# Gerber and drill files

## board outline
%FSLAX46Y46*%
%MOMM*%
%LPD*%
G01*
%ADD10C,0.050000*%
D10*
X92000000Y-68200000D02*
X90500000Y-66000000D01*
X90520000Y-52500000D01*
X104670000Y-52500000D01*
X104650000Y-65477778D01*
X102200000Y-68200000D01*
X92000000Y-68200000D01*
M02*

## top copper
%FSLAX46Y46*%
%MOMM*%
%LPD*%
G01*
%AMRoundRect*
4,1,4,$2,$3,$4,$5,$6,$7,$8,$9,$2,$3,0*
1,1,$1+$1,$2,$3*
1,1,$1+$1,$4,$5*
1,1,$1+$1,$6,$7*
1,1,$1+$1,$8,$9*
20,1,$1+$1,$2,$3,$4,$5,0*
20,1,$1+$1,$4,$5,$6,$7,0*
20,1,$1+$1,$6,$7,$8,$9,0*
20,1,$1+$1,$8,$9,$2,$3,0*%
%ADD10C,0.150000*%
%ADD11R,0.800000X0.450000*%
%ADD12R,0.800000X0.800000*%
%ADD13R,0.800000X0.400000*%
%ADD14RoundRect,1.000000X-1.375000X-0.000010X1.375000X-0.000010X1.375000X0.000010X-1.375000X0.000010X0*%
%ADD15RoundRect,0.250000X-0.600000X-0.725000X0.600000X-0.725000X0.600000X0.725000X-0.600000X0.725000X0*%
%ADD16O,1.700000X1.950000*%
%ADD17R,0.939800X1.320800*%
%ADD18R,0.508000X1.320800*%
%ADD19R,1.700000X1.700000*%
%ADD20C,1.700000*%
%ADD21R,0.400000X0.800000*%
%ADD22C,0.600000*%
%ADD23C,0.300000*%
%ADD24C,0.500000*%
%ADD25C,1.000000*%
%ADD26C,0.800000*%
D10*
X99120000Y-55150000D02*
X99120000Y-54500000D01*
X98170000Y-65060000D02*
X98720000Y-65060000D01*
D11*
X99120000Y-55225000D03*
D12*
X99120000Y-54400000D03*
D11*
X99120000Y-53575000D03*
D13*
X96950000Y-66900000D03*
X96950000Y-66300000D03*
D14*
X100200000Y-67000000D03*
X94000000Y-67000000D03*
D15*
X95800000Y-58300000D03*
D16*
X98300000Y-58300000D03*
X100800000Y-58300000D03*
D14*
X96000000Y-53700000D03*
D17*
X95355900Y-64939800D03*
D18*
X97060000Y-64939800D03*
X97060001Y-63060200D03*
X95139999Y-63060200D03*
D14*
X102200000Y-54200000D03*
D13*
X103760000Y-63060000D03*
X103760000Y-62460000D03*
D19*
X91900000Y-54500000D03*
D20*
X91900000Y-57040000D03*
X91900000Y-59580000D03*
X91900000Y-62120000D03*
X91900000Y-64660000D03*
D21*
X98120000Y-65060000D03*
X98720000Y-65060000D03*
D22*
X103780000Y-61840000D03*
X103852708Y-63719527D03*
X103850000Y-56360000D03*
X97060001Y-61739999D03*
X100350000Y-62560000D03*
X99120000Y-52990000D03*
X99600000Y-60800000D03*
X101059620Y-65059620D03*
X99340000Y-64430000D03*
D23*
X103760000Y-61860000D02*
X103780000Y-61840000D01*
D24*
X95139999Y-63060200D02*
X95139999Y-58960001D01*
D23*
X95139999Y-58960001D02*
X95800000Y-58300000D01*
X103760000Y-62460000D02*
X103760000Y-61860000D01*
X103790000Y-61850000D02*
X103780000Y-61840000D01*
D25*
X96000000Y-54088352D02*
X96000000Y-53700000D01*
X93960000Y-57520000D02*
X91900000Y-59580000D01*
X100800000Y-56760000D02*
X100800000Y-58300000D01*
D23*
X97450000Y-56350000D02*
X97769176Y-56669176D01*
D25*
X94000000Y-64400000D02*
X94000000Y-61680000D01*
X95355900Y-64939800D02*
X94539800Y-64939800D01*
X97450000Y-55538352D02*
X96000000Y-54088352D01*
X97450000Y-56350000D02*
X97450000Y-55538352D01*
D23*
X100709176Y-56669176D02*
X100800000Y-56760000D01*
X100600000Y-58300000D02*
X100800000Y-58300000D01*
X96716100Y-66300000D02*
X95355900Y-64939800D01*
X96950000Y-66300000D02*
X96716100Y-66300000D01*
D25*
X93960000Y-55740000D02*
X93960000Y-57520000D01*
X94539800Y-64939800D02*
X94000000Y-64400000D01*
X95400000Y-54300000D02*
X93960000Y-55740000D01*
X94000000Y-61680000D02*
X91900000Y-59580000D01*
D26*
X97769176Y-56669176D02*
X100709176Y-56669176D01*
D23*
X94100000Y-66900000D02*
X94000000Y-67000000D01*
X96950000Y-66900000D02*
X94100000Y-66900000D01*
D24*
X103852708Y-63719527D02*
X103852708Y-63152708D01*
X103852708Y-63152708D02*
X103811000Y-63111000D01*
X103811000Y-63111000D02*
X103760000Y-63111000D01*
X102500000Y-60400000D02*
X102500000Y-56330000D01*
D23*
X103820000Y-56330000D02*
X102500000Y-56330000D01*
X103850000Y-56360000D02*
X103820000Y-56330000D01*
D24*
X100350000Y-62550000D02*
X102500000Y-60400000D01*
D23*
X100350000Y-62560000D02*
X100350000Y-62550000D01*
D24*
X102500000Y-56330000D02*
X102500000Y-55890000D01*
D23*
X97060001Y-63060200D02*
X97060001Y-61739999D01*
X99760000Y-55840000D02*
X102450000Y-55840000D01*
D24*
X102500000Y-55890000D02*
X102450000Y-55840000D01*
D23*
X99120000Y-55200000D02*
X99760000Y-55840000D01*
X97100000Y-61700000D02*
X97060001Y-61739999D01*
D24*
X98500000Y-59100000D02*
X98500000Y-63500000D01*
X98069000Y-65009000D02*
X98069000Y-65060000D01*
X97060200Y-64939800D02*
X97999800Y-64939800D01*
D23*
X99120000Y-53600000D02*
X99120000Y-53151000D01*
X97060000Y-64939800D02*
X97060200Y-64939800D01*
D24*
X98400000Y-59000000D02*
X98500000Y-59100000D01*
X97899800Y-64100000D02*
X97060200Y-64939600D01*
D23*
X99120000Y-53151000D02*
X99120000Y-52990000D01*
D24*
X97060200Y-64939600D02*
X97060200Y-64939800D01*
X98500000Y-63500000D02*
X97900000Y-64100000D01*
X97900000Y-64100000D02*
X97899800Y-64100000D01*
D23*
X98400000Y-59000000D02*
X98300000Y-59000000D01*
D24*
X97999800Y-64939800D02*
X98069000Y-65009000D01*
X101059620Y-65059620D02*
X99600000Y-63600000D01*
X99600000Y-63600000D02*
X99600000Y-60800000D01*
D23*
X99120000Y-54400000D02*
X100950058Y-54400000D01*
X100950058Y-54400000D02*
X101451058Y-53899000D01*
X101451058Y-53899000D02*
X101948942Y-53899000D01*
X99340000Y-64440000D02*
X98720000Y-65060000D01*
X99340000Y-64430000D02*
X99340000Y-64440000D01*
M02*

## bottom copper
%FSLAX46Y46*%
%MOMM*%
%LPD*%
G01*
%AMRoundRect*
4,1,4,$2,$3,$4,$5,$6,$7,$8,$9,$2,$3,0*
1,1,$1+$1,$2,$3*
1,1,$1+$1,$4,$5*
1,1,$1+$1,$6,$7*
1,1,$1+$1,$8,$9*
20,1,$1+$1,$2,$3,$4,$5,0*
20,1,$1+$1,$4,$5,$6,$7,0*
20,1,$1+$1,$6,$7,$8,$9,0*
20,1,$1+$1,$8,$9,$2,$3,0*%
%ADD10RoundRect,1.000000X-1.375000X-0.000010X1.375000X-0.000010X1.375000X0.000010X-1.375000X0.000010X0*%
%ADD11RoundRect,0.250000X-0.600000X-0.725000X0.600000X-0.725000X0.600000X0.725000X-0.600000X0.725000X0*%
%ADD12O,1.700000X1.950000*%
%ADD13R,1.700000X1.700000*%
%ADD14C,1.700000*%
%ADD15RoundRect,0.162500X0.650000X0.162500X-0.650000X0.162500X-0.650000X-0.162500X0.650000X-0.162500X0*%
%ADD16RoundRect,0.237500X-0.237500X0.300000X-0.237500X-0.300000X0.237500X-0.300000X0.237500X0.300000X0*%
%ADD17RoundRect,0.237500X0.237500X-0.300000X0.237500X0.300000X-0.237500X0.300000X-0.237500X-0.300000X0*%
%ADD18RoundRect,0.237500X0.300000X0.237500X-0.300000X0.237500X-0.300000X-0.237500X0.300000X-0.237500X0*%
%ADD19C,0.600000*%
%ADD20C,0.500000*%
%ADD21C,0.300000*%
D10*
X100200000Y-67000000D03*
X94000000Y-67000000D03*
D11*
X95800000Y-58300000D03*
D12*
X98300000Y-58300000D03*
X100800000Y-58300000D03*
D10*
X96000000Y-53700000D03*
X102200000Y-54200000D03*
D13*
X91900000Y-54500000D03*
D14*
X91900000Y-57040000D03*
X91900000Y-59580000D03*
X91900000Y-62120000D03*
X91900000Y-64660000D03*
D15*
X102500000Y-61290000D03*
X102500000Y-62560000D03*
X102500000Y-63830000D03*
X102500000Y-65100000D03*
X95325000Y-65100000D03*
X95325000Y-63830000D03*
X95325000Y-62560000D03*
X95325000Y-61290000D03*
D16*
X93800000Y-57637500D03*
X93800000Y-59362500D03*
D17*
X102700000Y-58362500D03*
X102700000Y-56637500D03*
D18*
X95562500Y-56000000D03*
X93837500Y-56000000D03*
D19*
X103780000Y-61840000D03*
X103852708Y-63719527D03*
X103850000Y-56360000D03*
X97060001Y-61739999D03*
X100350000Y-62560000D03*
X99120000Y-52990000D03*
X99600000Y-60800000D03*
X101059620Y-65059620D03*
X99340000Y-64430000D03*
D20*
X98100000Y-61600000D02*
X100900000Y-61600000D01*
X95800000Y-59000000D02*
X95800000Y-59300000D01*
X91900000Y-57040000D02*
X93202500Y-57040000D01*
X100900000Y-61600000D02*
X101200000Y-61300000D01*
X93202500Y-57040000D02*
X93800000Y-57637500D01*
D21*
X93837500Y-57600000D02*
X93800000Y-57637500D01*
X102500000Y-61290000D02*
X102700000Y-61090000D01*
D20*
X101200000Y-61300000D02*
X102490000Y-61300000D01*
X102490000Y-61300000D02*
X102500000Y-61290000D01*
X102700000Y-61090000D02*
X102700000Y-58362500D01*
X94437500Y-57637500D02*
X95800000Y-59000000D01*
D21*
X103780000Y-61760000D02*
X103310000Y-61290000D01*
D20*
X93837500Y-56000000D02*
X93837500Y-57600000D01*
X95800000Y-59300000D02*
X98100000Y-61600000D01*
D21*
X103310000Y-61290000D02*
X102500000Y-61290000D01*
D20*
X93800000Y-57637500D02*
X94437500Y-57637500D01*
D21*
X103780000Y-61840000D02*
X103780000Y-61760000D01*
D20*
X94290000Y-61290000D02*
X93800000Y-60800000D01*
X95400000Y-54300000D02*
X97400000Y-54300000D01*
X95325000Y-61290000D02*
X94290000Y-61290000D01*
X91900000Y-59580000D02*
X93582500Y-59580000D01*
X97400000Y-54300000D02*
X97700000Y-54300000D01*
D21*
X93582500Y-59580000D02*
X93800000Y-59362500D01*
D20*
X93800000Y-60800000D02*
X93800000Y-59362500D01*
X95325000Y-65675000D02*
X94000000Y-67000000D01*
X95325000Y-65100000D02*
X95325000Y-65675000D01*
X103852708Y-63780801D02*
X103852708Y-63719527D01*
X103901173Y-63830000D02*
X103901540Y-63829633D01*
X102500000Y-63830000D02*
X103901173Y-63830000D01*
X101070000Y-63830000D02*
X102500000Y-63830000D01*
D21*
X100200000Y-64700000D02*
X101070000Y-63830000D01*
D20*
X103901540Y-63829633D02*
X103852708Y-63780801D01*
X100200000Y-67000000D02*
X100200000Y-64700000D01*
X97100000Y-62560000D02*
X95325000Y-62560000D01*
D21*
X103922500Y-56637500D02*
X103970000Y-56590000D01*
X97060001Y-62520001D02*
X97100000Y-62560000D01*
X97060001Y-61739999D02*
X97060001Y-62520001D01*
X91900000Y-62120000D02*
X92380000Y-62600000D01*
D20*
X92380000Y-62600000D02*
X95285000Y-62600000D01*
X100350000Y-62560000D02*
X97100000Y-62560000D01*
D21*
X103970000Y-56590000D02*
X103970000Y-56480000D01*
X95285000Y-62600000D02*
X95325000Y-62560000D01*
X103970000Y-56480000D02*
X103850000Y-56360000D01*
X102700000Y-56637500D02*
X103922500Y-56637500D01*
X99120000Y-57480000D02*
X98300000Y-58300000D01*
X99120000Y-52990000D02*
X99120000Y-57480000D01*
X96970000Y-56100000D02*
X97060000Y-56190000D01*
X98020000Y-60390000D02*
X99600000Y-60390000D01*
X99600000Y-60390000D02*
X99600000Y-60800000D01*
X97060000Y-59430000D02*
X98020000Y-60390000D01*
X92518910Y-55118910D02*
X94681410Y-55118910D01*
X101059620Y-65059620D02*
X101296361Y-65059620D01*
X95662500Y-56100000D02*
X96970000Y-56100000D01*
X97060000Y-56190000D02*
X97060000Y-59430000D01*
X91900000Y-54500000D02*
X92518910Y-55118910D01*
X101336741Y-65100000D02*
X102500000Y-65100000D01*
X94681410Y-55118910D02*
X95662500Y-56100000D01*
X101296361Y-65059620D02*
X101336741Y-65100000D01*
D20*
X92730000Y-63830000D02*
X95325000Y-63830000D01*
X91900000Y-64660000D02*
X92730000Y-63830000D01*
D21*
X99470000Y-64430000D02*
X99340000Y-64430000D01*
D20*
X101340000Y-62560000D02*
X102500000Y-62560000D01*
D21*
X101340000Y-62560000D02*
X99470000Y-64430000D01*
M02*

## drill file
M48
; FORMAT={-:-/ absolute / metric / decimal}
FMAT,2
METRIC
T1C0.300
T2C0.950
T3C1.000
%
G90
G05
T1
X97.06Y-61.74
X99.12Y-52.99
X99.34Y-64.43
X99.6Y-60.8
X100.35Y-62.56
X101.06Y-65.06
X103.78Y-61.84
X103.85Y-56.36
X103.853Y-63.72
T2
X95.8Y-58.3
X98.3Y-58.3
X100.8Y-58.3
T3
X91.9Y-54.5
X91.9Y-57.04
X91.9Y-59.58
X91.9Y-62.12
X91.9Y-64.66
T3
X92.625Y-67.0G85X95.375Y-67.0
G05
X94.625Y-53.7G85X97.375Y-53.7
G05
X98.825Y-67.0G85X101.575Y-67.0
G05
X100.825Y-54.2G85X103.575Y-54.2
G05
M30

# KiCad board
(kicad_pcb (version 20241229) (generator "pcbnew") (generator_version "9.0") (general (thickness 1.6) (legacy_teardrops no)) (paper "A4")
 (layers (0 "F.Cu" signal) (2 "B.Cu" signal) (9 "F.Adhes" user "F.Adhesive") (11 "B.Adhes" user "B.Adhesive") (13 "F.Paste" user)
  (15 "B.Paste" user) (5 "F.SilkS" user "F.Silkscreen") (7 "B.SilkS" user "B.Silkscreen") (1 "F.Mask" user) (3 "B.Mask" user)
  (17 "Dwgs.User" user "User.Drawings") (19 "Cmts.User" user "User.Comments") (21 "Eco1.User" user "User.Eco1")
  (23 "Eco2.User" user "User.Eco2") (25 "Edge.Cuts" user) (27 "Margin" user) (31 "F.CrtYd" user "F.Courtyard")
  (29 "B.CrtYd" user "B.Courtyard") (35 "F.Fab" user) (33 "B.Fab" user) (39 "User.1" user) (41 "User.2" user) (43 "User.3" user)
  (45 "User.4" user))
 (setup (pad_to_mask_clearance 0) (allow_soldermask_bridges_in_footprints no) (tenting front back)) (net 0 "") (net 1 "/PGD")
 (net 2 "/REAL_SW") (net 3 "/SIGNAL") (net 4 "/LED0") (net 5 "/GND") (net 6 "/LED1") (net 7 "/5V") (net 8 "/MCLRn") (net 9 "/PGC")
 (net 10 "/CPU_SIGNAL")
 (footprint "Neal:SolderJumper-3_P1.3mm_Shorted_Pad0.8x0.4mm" (layer "F.Cu") (at 99.12 54.4 90)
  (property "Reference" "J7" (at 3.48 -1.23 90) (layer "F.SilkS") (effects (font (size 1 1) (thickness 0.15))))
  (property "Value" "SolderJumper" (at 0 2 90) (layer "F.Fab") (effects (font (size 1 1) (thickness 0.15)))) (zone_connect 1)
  (fp_line (start -0.75 0) (end -0.1 0) (stroke (width 0.15) (type solid)) (layer "F.Cu"))
  (pad "1" smd rect (at -0.825 0 90) (size 0.45 0.8) (layers "F.Cu" "F.Mask") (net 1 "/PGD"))
  (pad "2" smd rect (at 0 0 90) (size 0.8 0.8) (layers "F.Cu" "F.Mask") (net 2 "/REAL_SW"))
  (pad "3" smd rect (at 0.825 0 90) (size 0.45 0.8) (layers "F.Cu" "F.Mask") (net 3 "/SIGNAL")))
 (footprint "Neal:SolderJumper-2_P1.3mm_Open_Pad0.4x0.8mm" (layer "F.Cu") (at 96.95 66.6 90)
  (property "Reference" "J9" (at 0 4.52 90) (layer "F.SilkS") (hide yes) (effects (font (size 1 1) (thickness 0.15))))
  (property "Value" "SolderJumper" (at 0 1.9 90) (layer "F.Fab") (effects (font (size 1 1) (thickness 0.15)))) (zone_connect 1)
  (pad "1" smd rect (at -0.3 0 90) (size 0.4 0.8) (layers "F.Cu" "F.Mask") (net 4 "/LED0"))
  (pad "2" smd rect (at 0.3 0 90) (size 0.4 0.8) (layers "F.Cu" "F.Mask") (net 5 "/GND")))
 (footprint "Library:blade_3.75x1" (layer "F.Cu") (at 100.2 67)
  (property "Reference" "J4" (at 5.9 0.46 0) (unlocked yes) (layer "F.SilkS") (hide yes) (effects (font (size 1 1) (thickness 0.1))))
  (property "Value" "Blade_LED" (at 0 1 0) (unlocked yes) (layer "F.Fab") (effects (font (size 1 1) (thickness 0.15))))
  (pad "1" thru_hole roundrect (at 0 0) (size 4.75 2) (drill oval 3.75 1) (layers "*.Cu" "*.Mask") (remove_unused_layers no)
   (roundrect_rratio 0.5) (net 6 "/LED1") (thermal_bridge_angle 45)))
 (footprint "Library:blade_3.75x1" (layer "F.Cu") (at 94 67)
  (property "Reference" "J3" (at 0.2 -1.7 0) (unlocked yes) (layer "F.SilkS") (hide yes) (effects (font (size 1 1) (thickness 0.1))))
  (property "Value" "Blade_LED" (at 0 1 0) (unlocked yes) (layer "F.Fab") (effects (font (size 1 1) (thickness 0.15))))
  (pad "1" thru_hole roundrect (at 0 0) (size 4.75 2) (drill oval 3.75 1) (layers "*.Cu" "*.Mask") (remove_unused_layers no)
   (roundrect_rratio 0.5) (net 4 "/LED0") (thermal_bridge_angle 45)))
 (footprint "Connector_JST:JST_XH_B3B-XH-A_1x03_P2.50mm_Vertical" (layer "F.Cu") (at 95.8 58.3)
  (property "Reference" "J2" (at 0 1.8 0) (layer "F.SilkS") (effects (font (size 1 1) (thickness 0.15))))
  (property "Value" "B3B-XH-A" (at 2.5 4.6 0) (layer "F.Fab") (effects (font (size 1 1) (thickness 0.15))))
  (pad "1" thru_hole roundrect (at 0 0) (size 1.7 1.95) (drill 0.95) (layers "*.Cu" "*.Mask") (remove_unused_layers no)
   (roundrect_rratio 0.147059) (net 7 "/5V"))
  (pad "2" thru_hole oval (at 2.5 0) (size 1.7 1.95) (drill 0.95) (layers "*.Cu" "*.Mask") (remove_unused_layers no) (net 3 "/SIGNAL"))
  (pad "3" thru_hole oval (at 5 0) (size 1.7 1.95) (drill 0.95) (layers "*.Cu" "*.Mask") (remove_unused_layers no) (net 5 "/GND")))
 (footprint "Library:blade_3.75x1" (layer "F.Cu") (at 95.4 54.3)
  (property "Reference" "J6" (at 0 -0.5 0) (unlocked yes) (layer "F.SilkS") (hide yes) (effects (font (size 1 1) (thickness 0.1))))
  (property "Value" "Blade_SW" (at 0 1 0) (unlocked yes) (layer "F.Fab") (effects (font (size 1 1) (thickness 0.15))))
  (pad "1" thru_hole roundrect (at 0.6 -0.6) (size 4.75 2) (drill oval 3.75 1) (layers "*.Cu" "*.Mask") (remove_unused_layers no)
   (roundrect_rratio 0.5) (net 5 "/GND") (thermal_bridge_angle 45)))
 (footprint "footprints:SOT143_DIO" (layer "F.Cu") (at 96.1 64)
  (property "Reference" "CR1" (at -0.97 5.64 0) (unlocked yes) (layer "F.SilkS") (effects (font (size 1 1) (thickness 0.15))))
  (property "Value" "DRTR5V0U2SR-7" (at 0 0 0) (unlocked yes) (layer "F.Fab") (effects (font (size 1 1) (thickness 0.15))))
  (pad "1" smd rect (at -0.7441 0.9398) (size 0.9398 1.3208) (layers "F.Cu" "F.Mask" "F.Paste") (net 5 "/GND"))
  (pad "2" smd rect (at 0.96 0.9398) (size 0.508 1.3208) (layers "F.Cu" "F.Mask" "F.Paste") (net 3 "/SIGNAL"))
  (pad "3" smd rect (at 0.960001 -0.9398) (size 0.508 1.3208) (layers "F.Cu" "F.Mask" "F.Paste") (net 1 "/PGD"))
  (pad "4" smd rect (at -0.960001 -0.9398) (size 0.508 1.3208) (layers "F.Cu" "F.Mask" "F.Paste") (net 7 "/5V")))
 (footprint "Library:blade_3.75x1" (layer "F.Cu") (at 101.7 55.5)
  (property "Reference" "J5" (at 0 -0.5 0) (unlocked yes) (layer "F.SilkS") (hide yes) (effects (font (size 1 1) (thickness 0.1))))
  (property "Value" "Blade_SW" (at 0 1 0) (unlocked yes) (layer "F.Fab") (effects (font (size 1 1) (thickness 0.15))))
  (pad "1" thru_hole roundrect (at 0.5 -1.3) (size 4.75 2) (drill oval 3.75 1) (layers "*.Cu" "*.Mask") (remove_unused_layers no)
   (roundrect_rratio 0.5) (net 2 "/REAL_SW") (thermal_bridge_angle 45)))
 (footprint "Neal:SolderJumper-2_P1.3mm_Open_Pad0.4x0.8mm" (layer "F.Cu") (at 103.76 62.76 90)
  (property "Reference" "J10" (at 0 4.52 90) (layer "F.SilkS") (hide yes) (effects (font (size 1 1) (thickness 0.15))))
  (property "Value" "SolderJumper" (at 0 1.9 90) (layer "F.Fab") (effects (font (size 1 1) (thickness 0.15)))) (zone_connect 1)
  (pad "1" smd rect (at -0.3 0 90) (size 0.4 0.8) (layers "F.Cu" "F.Mask") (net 6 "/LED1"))
  (pad "2" smd rect (at 0.3 0 90) (size 0.4 0.8) (layers "F.Cu" "F.Mask") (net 7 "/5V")))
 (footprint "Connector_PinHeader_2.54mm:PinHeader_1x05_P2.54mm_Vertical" (layer "F.Cu") (at 91.9 54.5)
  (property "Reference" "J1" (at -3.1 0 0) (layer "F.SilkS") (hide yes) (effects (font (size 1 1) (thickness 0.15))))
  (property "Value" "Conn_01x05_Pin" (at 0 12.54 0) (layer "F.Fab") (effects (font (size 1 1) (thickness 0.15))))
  (pad "1" thru_hole rect (at 0 0) (size 1.7 1.7) (drill 1) (layers "*.Cu" "*.Mask") (remove_unused_layers no) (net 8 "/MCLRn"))
  (pad "2" thru_hole circle (at 0 2.54) (size 1.7 1.7) (drill 1) (layers "*.Cu" "*.Mask") (remove_unused_layers no) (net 7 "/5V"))
  (pad "3" thru_hole circle (at 0 5.08) (size 1.7 1.7) (drill 1) (layers "*.Cu" "*.Mask") (remove_unused_layers no) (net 5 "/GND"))
  (pad "4" thru_hole circle (at 0 7.62) (size 1.7 1.7) (drill 1) (layers "*.Cu" "*.Mask") (remove_unused_layers no) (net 1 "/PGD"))
  (pad "5" thru_hole circle (at 0 10.16) (size 1.7 1.7) (drill 1) (layers "*.Cu" "*.Mask") (remove_unused_layers no) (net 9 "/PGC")))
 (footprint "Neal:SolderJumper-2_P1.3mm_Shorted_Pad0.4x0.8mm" (layer "F.Cu") (at 98.42 65.06)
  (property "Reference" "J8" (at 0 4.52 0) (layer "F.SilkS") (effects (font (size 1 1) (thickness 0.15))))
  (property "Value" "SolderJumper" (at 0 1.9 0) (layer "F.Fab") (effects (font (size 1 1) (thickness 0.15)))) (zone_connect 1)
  (fp_line (start -0.25 0) (end 0.3 0) (stroke (width 0.15) (type solid)) (layer "F.Cu"))
  (pad "1" smd rect (at -0.3 0) (size 0.4 0.8) (layers "F.Cu" "F.Mask") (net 3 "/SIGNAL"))
  (pad "2" smd rect (at 0.3 0) (size 0.4 0.8) (layers "F.Cu" "F.Mask") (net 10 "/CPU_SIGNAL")))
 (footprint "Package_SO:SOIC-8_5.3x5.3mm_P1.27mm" (layer "B.Cu") (at 98.9125 63.195 180)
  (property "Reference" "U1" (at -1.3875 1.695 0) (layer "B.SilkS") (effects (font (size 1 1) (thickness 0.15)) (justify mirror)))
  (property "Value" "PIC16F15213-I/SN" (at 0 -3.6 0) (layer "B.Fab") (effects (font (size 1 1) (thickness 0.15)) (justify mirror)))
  (pad "1" smd roundrect (at -3.5875 1.905 180) (size 1.625 0.65) (layers "B.Cu" "B.Mask" "B.Paste") (roundrect_rratio 0.25) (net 7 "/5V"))
  (pad "2" smd roundrect (at -3.5875 0.635 180) (size 1.625 0.65) (layers "B.Cu" "B.Mask" "B.Paste") (roundrect_rratio 0.25)
   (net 10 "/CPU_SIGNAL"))
  (pad "3" smd roundrect (at -3.5875 -0.635 180) (size 1.625 0.65) (layers "B.Cu" "B.Mask" "B.Paste") (roundrect_rratio 0.25)
   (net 6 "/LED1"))
  (pad "4" smd roundrect (at -3.5875 -1.905 180) (size 1.625 0.65) (layers "B.Cu" "B.Mask" "B.Paste") (roundrect_rratio 0.25)
   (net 8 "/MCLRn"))
  (pad "5" smd roundrect (at 3.5875 -1.905 180) (size 1.625 0.65) (layers "B.Cu" "B.Mask" "B.Paste") (roundrect_rratio 0.25) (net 4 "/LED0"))
  (pad "6" smd roundrect (at 3.5875 -0.635 180) (size 1.625 0.65) (layers "B.Cu" "B.Mask" "B.Paste") (roundrect_rratio 0.25) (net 9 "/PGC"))
  (pad "7" smd roundrect (at 3.5875 0.635 180) (size 1.625 0.65) (layers "B.Cu" "B.Mask" "B.Paste") (roundrect_rratio 0.25) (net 1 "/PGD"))
  (pad "8" smd roundrect (at 3.5875 1.905 180) (size 1.625 0.65) (layers "B.Cu" "B.Mask" "B.Paste") (roundrect_rratio 0.25) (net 5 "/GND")))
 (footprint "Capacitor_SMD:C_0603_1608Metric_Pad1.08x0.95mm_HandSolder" (layer "B.Cu") (at 93.8 58.5 -90)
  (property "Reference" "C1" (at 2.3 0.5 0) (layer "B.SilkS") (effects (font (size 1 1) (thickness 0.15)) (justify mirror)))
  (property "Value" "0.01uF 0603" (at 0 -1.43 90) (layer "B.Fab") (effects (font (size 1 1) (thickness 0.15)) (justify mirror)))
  (pad "1" smd roundrect (at -0.8625 0 270) (size 1.075 0.95) (layers "B.Cu" "B.Mask" "B.Paste") (roundrect_rratio 0.25) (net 7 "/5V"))
  (pad "2" smd roundrect (at 0.8625 0 270) (size 1.075 0.95) (layers "B.Cu" "B.Mask" "B.Paste") (roundrect_rratio 0.25) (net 5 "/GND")))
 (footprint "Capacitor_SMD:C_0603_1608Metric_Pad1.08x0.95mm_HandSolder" (layer "B.Cu") (at 102.7 57.5 90)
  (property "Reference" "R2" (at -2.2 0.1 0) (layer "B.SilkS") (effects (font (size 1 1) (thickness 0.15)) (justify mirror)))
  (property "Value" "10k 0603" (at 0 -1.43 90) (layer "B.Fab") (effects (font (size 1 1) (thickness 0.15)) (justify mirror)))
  (pad "1" smd roundrect (at -0.8625 0 90) (size 1.075 0.95) (layers "B.Cu" "B.Mask" "B.Paste") (roundrect_rratio 0.25) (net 7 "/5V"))
  (pad "2" smd roundrect (at 0.8625 0 90) (size 1.075 0.95) (layers "B.Cu" "B.Mask" "B.Paste") (roundrect_rratio 0.25) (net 1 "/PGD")))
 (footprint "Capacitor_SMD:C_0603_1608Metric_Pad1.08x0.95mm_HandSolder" (layer "B.Cu") (at 94.7 56 180)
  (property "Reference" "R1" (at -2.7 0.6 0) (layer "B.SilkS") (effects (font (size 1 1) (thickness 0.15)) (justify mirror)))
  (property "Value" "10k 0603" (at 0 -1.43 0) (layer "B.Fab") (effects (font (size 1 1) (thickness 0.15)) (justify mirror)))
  (pad "1" smd roundrect (at -0.8625 0 180) (size 1.075 0.95) (layers "B.Cu" "B.Mask" "B.Paste") (roundrect_rratio 0.25) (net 8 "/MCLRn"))
  (pad "2" smd roundrect (at 0.8625 0 180) (size 1.075 0.95) (layers "B.Cu" "B.Mask" "B.Paste") (roundrect_rratio 0.25) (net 7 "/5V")))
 (gr_poly
  (pts (xy 92 68.2) (xy 90.5 66) (xy 90.52 52.5) (xy 104.67 52.5) (xy 104.65 65.477778) (xy 102.2 68.2)) (stroke (width 0.05) (type solid))
  (fill no) (layer "Edge.Cuts"))
 (segment (start 103.76 61.86) (end 103.78 61.84) (width 0.3) (layer "F.Cu") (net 7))
 (segment (start 95.139999 63.0602) (end 95.139999 58.960001) (width 0.5) (layer "F.Cu") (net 7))
 (segment (start 95.139999 58.960001) (end 95.8 58.3) (width 0.3) (layer "F.Cu") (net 7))
 (segment (start 103.76 62.46) (end 103.76 61.86) (width 0.3) (layer "F.Cu") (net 7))
 (segment (start 103.79 61.85) (end 103.78 61.84) (width 0.3) (layer "F.Cu") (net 7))
 (via (at 103.78 61.84) (size 0.6) (drill 0.3) (layers "F.Cu" "B.Cu") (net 7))
 (segment (start 98.1 61.6) (end 100.9 61.6) (width 0.5) (layer "B.Cu") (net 7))
 (segment (start 95.8 59) (end 95.8 59.3) (width 0.5) (layer "B.Cu") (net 7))
 (segment (start 91.9 57.04) (end 93.2025 57.04) (width 0.5) (layer "B.Cu") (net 7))
 (segment (start 100.9 61.6) (end 101.2 61.3) (width 0.5) (layer "B.Cu") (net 7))
 (segment (start 93.2025 57.04) (end 93.8 57.6375) (width 0.5) (layer "B.Cu") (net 7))
 (segment (start 93.8375 57.6) (end 93.8 57.6375) (width 0.3) (layer "B.Cu") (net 7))
 (segment (start 102.5 61.29) (end 102.7 61.09) (width 0.3) (layer "B.Cu") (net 7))
 (segment (start 101.2 61.3) (end 102.49 61.3) (width 0.5) (layer "B.Cu") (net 7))
 (segment (start 102.49 61.3) (end 102.5 61.29) (width 0.5) (layer "B.Cu") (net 7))
 (segment (start 102.7 61.09) (end 102.7 58.3625) (width 0.5) (layer "B.Cu") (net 7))
 (segment (start 94.4375 57.6375) (end 95.8 59) (width 0.5) (layer "B.Cu") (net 7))
 (segment (start 103.78 61.76) (end 103.31 61.29) (width 0.3) (layer "B.Cu") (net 7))
 (segment (start 93.8375 56) (end 93.8375 57.6) (width 0.5) (layer "B.Cu") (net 7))
 (segment (start 95.8 59.3) (end 98.1 61.6) (width 0.5) (layer "B.Cu") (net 7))
 (segment (start 103.31 61.29) (end 102.5 61.29) (width 0.3) (layer "B.Cu") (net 7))
 (segment (start 93.8 57.6375) (end 94.4375 57.6375) (width 0.5) (layer "B.Cu") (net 7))
 (segment (start 103.78 61.84) (end 103.78 61.76) (width 0.3) (layer "B.Cu") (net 7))
 (segment (start 96 54.088352) (end 96 53.7) (width 1) (layer "F.Cu") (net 5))
 (segment (start 93.96 57.52) (end 91.9 59.58) (width 1) (layer "F.Cu") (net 5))
 (segment (start 100.8 56.76) (end 100.8 58.3) (width 1) (layer "F.Cu") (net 5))
 (segment (start 97.45 56.35) (end 97.769176 56.669176) (width 0.3) (layer "F.Cu") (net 5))
 (segment (start 94 64.4) (end 94 61.68) (width 1) (layer "F.Cu") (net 5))
 (segment (start 95.3559 64.9398) (end 94.5398 64.9398) (width 1) (layer "F.Cu") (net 5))
 (segment (start 97.45 55.538352) (end 96 54.088352) (width 1) (layer "F.Cu") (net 5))
 (segment (start 97.45 56.35) (end 97.45 55.538352) (width 1) (layer "F.Cu") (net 5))
 (segment (start 100.709176 56.669176) (end 100.8 56.76) (width 0.3) (layer "F.Cu") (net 5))
 (segment (start 100.6 58.3) (end 100.8 58.3) (width 0.3) (layer "F.Cu") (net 5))
 (segment (start 96.7161 66.3) (end 95.3559 64.9398) (width 0.3) (layer "F.Cu") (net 5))
 (segment (start 96.95 66.3) (end 96.7161 66.3) (width 0.3) (layer "F.Cu") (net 5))
 (segment (start 93.96 55.74) (end 93.96 57.52) (width 1) (layer "F.Cu") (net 5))
 (segment (start 94.5398 64.9398) (end 94 64.4) (width 1) (layer "F.Cu") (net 5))
 (segment (start 95.4 54.3) (end 93.96 55.74) (width 1) (layer "F.Cu") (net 5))
 (segment (start 94 61.68) (end 91.9 59.58) (width 1) (layer "F.Cu") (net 5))
 (segment (start 97.769176 56.669176) (end 100.709176 56.669176) (width 0.8) (layer "F.Cu") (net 5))
 (segment (start 94.29 61.29) (end 93.8 60.8) (width 0.5) (layer "B.Cu") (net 5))
 (segment (start 95.4 54.3) (end 97.4 54.3) (width 0.5) (layer "B.Cu") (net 5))
 (segment (start 95.325 61.29) (end 94.29 61.29) (width 0.5) (layer "B.Cu") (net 5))
 (segment (start 91.9 59.58) (end 93.5825 59.58) (width 0.5) (layer "B.Cu") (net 5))
 (segment (start 97.4 54.3) (end 97.7 54.3) (width 0.5) (layer "B.Cu") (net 5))
 (segment (start 93.5825 59.58) (end 93.8 59.3625) (width 0.3) (layer "B.Cu") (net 5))
 (segment (start 93.8 60.8) (end 93.8 59.3625) (width 0.5) (layer "B.Cu") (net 5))
 (segment (start 94.1 66.9) (end 94 67) (width 0.3) (layer "F.Cu") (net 4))
 (segment (start 96.95 66.9) (end 94.1 66.9) (width 0.3) (layer "F.Cu") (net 4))
 (segment (start 95.325 65.675) (end 94 67) (width 0.5) (layer "B.Cu") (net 4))
 (segment (start 95.325 65.1) (end 95.325 65.675) (width 0.5) (layer "B.Cu") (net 4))
 (segment (start 103.852708 63.719527) (end 103.852708 63.152708) (width 0.5) (layer "F.Cu") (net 6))
 (segment (start 103.852708 63.152708) (end 103.811 63.111) (width 0.5) (layer "F.Cu") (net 6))
 (segment (start 103.811 63.111) (end 103.76 63.111) (width 0.5) (layer "F.Cu") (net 6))
 (via (at 103.852708 63.719527) (size 0.6) (drill 0.3) (layers "F.Cu" "B.Cu") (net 6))
 (segment (start 103.852708 63.780801) (end 103.852708 63.719527) (width 0.5) (layer "B.Cu") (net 6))
 (segment (start 103.901173 63.83) (end 103.90154 63.829633) (width 0.5) (layer "B.Cu") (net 6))
 (segment (start 102.5 63.83) (end 103.901173 63.83) (width 0.5) (layer "B.Cu") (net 6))
 (segment (start 101.07 63.83) (end 102.5 63.83) (width 0.5) (layer "B.Cu") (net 6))
 (segment (start 100.2 64.7) (end 101.07 63.83) (width 0.3) (layer "B.Cu") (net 6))
 (segment (start 103.90154 63.829633) (end 103.852708 63.780801) (width 0.5) (layer "B.Cu") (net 6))
 (segment (start 100.2 67) (end 100.2 64.7) (width 0.5) (layer "B.Cu") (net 6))
 (segment (start 102.5 60.4) (end 102.5 56.33) (width 0.5) (layer "F.Cu") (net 1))
 (segment (start 103.82 56.33) (end 102.5 56.33) (width 0.3) (layer "F.Cu") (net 1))
 (segment (start 103.85 56.36) (end 103.82 56.33) (width 0.3) (layer "F.Cu") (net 1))
 (segment (start 100.35 62.55) (end 102.5 60.4) (width 0.5) (layer "F.Cu") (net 1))
 (segment (start 100.35 62.56) (end 100.35 62.55) (width 0.3) (layer "F.Cu") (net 1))
 (segment (start 102.5 56.33) (end 102.5 55.89) (width 0.5) (layer "F.Cu") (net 1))
 (segment (start 97.060001 63.0602) (end 97.060001 61.739999) (width 0.3) (layer "F.Cu") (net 1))
 (segment (start 99.76 55.84) (end 102.45 55.84) (width 0.3) (layer "F.Cu") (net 1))
 (segment (start 102.5 55.89) (end 102.45 55.84) (width 0.5) (layer "F.Cu") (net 1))
 (segment (start 99.12 55.2) (end 99.76 55.84) (width 0.3) (layer "F.Cu") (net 1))
 (segment (start 97.1 61.7) (end 97.060001 61.739999) (width 0.3) (layer "F.Cu") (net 1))
 (via (at 103.85 56.36) (size 0.6) (drill 0.3) (layers "F.Cu" "B.Cu") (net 1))
 (via (at 97.060001 61.739999) (size 0.6) (drill 0.3) (layers "F.Cu" "B.Cu") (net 1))
 (via (at 100.35 62.56) (size 0.6) (drill 0.3) (layers "F.Cu" "B.Cu") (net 1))
 (segment (start 97.1 62.56) (end 95.325 62.56) (width 0.5) (layer "B.Cu") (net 1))
 (segment (start 103.9225 56.6375) (end 103.97 56.59) (width 0.3) (layer "B.Cu") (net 1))
 (segment (start 97.060001 62.520001) (end 97.1 62.56) (width 0.3) (layer "B.Cu") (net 1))
 (segment (start 97.060001 61.739999) (end 97.060001 62.520001) (width 0.3) (layer "B.Cu") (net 1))
 (segment (start 91.9 62.12) (end 92.38 62.6) (width 0.3) (layer "B.Cu") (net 1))
 (segment (start 92.38 62.6) (end 95.285 62.6) (width 0.5) (layer "B.Cu") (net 1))
 (segment (start 100.35 62.56) (end 97.1 62.56) (width 0.5) (layer "B.Cu") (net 1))
 (segment (start 103.97 56.59) (end 103.97 56.48) (width 0.3) (layer "B.Cu") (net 1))
 (segment (start 95.285 62.6) (end 95.325 62.56) (width 0.3) (layer "B.Cu") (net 1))
 (segment (start 103.97 56.48) (end 103.85 56.36) (width 0.3) (layer "B.Cu") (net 1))
 (segment (start 102.7 56.6375) (end 103.9225 56.6375) (width 0.3) (layer "B.Cu") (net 1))
 (segment (start 98.5 59.1) (end 98.5 63.5) (width 0.5) (layer "F.Cu") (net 3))
 (segment (start 98.069 65.009) (end 98.069 65.06) (width 0.5) (layer "F.Cu") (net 3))
 (segment (start 97.0602 64.9398) (end 97.9998 64.9398) (width 0.5) (layer "F.Cu") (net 3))
 (segment (start 99.12 53.6) (end 99.12 53.151) (width 0.3) (layer "F.Cu") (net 3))
 (segment (start 97.06 64.9398) (end 97.0602 64.9398) (width 0.3) (layer "F.Cu") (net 3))
 (segment (start 98.4 59) (end 98.5 59.1) (width 0.5) (layer "F.Cu") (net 3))
 (segment (start 97.8998 64.1) (end 97.0602 64.9396) (width 0.5) (layer "F.Cu") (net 3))
 (segment (start 99.12 53.151) (end 99.12 52.99) (width 0.3) (layer "F.Cu") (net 3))
 (segment (start 97.0602 64.9396) (end 97.0602 64.9398) (width 0.5) (layer "F.Cu") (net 3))
 (segment (start 98.5 63.5) (end 97.9 64.1) (width 0.5) (layer "F.Cu") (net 3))
 (segment (start 97.9 64.1) (end 97.8998 64.1) (width 0.5) (layer "F.Cu") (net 3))
 (segment (start 98.4 59) (end 98.3 59) (width 0.3) (layer "F.Cu") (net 3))
 (segment (start 97.9998 64.9398) (end 98.069 65.009) (width 0.5) (layer "F.Cu") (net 3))
 (via (at 99.12 52.99) (size 0.6) (drill 0.3) (layers "F.Cu" "B.Cu") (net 3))
 (segment (start 99.12 57.48) (end 98.3 58.3) (width 0.3) (layer "B.Cu") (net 3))
 (segment (start 99.12 52.99) (end 99.12 57.48) (width 0.3) (layer "B.Cu") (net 3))
 (segment (start 101.05962 65.05962) (end 99.6 63.6) (width 0.5) (layer "F.Cu") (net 8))
 (segment (start 99.6 63.6) (end 99.6 60.8) (width 0.5) (layer "F.Cu") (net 8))
 (via (at 99.6 60.8) (size 0.6) (drill 0.3) (layers "F.Cu" "B.Cu") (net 8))
 (via (at 101.05962 65.05962) (size 0.6) (drill 0.3) (layers "F.Cu" "B.Cu") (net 8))
 (segment (start 96.97 56.1) (end 97.06 56.19) (width 0.3) (layer "B.Cu") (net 8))
 (segment (start 98.02 60.39) (end 99.6 60.39) (width 0.3) (layer "B.Cu") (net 8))
 (segment (start 99.6 60.39) (end 99.6 60.8) (width 0.3) (layer "B.Cu") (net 8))
 (segment (start 97.06 59.43) (end 98.02 60.39) (width 0.3) (layer "B.Cu") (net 8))
 (segment (start 92.51891 55.11891) (end 94.68141 55.11891) (width 0.3) (layer "B.Cu") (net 8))
 (segment (start 101.05962 65.05962) (end 101.296361 65.05962) (width 0.3) (layer "B.Cu") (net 8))
 (segment (start 95.6625 56.1) (end 96.97 56.1) (width 0.3) (layer "B.Cu") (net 8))
 (segment (start 97.06 56.19) (end 97.06 59.43) (width 0.3) (layer "B.Cu") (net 8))
 (segment (start 91.9 54.5) (end 92.51891 55.11891) (width 0.3) (layer "B.Cu") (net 8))
 (segment (start 101.336741 65.1) (end 102.5 65.1) (width 0.3) (layer "B.Cu") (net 8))
 (segment (start 94.68141 55.11891) (end 95.6625 56.1) (width 0.3) (layer "B.Cu") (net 8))
 (segment (start 101.296361 65.05962) (end 101.336741 65.1) (width 0.3) (layer "B.Cu") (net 8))
 (segment (start 92.73 63.83) (end 95.325 63.83) (width 0.5) (layer "B.Cu") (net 9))
 (segment (start 91.9 64.66) (end 92.73 63.83) (width 0.5) (layer "B.Cu") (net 9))
 (segment (start 99.12 54.4) (end 100.950058 54.4) (width 0.3) (layer "F.Cu") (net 2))
 (segment (start 100.950058 54.4) (end 101.451058 53.899) (width 0.3) (layer "F.Cu") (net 2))
 (segment (start 101.451058 53.899) (end 101.948942 53.899) (width 0.3) (layer "F.Cu") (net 2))
 (segment (start 99.34 64.44) (end 98.72 65.06) (width 0.3) (layer "F.Cu") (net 10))
 (segment (start 99.34 64.43) (end 99.34 64.44) (width 0.3) (layer "F.Cu") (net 10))
 (via (at 99.34 64.43) (size 0.6) (drill 0.3) (layers "F.Cu" "B.Cu") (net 10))
 (segment (start 99.47 64.43) (end 99.34 64.43) (width 0.3) (layer "B.Cu") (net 10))
 (segment (start 101.34 62.56) (end 102.5 62.56) (width 0.5) (layer "B.Cu") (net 10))
 (segment (start 101.34 62.56) (end 99.47 64.43) (width 0.3) (layer "B.Cu") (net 10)))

